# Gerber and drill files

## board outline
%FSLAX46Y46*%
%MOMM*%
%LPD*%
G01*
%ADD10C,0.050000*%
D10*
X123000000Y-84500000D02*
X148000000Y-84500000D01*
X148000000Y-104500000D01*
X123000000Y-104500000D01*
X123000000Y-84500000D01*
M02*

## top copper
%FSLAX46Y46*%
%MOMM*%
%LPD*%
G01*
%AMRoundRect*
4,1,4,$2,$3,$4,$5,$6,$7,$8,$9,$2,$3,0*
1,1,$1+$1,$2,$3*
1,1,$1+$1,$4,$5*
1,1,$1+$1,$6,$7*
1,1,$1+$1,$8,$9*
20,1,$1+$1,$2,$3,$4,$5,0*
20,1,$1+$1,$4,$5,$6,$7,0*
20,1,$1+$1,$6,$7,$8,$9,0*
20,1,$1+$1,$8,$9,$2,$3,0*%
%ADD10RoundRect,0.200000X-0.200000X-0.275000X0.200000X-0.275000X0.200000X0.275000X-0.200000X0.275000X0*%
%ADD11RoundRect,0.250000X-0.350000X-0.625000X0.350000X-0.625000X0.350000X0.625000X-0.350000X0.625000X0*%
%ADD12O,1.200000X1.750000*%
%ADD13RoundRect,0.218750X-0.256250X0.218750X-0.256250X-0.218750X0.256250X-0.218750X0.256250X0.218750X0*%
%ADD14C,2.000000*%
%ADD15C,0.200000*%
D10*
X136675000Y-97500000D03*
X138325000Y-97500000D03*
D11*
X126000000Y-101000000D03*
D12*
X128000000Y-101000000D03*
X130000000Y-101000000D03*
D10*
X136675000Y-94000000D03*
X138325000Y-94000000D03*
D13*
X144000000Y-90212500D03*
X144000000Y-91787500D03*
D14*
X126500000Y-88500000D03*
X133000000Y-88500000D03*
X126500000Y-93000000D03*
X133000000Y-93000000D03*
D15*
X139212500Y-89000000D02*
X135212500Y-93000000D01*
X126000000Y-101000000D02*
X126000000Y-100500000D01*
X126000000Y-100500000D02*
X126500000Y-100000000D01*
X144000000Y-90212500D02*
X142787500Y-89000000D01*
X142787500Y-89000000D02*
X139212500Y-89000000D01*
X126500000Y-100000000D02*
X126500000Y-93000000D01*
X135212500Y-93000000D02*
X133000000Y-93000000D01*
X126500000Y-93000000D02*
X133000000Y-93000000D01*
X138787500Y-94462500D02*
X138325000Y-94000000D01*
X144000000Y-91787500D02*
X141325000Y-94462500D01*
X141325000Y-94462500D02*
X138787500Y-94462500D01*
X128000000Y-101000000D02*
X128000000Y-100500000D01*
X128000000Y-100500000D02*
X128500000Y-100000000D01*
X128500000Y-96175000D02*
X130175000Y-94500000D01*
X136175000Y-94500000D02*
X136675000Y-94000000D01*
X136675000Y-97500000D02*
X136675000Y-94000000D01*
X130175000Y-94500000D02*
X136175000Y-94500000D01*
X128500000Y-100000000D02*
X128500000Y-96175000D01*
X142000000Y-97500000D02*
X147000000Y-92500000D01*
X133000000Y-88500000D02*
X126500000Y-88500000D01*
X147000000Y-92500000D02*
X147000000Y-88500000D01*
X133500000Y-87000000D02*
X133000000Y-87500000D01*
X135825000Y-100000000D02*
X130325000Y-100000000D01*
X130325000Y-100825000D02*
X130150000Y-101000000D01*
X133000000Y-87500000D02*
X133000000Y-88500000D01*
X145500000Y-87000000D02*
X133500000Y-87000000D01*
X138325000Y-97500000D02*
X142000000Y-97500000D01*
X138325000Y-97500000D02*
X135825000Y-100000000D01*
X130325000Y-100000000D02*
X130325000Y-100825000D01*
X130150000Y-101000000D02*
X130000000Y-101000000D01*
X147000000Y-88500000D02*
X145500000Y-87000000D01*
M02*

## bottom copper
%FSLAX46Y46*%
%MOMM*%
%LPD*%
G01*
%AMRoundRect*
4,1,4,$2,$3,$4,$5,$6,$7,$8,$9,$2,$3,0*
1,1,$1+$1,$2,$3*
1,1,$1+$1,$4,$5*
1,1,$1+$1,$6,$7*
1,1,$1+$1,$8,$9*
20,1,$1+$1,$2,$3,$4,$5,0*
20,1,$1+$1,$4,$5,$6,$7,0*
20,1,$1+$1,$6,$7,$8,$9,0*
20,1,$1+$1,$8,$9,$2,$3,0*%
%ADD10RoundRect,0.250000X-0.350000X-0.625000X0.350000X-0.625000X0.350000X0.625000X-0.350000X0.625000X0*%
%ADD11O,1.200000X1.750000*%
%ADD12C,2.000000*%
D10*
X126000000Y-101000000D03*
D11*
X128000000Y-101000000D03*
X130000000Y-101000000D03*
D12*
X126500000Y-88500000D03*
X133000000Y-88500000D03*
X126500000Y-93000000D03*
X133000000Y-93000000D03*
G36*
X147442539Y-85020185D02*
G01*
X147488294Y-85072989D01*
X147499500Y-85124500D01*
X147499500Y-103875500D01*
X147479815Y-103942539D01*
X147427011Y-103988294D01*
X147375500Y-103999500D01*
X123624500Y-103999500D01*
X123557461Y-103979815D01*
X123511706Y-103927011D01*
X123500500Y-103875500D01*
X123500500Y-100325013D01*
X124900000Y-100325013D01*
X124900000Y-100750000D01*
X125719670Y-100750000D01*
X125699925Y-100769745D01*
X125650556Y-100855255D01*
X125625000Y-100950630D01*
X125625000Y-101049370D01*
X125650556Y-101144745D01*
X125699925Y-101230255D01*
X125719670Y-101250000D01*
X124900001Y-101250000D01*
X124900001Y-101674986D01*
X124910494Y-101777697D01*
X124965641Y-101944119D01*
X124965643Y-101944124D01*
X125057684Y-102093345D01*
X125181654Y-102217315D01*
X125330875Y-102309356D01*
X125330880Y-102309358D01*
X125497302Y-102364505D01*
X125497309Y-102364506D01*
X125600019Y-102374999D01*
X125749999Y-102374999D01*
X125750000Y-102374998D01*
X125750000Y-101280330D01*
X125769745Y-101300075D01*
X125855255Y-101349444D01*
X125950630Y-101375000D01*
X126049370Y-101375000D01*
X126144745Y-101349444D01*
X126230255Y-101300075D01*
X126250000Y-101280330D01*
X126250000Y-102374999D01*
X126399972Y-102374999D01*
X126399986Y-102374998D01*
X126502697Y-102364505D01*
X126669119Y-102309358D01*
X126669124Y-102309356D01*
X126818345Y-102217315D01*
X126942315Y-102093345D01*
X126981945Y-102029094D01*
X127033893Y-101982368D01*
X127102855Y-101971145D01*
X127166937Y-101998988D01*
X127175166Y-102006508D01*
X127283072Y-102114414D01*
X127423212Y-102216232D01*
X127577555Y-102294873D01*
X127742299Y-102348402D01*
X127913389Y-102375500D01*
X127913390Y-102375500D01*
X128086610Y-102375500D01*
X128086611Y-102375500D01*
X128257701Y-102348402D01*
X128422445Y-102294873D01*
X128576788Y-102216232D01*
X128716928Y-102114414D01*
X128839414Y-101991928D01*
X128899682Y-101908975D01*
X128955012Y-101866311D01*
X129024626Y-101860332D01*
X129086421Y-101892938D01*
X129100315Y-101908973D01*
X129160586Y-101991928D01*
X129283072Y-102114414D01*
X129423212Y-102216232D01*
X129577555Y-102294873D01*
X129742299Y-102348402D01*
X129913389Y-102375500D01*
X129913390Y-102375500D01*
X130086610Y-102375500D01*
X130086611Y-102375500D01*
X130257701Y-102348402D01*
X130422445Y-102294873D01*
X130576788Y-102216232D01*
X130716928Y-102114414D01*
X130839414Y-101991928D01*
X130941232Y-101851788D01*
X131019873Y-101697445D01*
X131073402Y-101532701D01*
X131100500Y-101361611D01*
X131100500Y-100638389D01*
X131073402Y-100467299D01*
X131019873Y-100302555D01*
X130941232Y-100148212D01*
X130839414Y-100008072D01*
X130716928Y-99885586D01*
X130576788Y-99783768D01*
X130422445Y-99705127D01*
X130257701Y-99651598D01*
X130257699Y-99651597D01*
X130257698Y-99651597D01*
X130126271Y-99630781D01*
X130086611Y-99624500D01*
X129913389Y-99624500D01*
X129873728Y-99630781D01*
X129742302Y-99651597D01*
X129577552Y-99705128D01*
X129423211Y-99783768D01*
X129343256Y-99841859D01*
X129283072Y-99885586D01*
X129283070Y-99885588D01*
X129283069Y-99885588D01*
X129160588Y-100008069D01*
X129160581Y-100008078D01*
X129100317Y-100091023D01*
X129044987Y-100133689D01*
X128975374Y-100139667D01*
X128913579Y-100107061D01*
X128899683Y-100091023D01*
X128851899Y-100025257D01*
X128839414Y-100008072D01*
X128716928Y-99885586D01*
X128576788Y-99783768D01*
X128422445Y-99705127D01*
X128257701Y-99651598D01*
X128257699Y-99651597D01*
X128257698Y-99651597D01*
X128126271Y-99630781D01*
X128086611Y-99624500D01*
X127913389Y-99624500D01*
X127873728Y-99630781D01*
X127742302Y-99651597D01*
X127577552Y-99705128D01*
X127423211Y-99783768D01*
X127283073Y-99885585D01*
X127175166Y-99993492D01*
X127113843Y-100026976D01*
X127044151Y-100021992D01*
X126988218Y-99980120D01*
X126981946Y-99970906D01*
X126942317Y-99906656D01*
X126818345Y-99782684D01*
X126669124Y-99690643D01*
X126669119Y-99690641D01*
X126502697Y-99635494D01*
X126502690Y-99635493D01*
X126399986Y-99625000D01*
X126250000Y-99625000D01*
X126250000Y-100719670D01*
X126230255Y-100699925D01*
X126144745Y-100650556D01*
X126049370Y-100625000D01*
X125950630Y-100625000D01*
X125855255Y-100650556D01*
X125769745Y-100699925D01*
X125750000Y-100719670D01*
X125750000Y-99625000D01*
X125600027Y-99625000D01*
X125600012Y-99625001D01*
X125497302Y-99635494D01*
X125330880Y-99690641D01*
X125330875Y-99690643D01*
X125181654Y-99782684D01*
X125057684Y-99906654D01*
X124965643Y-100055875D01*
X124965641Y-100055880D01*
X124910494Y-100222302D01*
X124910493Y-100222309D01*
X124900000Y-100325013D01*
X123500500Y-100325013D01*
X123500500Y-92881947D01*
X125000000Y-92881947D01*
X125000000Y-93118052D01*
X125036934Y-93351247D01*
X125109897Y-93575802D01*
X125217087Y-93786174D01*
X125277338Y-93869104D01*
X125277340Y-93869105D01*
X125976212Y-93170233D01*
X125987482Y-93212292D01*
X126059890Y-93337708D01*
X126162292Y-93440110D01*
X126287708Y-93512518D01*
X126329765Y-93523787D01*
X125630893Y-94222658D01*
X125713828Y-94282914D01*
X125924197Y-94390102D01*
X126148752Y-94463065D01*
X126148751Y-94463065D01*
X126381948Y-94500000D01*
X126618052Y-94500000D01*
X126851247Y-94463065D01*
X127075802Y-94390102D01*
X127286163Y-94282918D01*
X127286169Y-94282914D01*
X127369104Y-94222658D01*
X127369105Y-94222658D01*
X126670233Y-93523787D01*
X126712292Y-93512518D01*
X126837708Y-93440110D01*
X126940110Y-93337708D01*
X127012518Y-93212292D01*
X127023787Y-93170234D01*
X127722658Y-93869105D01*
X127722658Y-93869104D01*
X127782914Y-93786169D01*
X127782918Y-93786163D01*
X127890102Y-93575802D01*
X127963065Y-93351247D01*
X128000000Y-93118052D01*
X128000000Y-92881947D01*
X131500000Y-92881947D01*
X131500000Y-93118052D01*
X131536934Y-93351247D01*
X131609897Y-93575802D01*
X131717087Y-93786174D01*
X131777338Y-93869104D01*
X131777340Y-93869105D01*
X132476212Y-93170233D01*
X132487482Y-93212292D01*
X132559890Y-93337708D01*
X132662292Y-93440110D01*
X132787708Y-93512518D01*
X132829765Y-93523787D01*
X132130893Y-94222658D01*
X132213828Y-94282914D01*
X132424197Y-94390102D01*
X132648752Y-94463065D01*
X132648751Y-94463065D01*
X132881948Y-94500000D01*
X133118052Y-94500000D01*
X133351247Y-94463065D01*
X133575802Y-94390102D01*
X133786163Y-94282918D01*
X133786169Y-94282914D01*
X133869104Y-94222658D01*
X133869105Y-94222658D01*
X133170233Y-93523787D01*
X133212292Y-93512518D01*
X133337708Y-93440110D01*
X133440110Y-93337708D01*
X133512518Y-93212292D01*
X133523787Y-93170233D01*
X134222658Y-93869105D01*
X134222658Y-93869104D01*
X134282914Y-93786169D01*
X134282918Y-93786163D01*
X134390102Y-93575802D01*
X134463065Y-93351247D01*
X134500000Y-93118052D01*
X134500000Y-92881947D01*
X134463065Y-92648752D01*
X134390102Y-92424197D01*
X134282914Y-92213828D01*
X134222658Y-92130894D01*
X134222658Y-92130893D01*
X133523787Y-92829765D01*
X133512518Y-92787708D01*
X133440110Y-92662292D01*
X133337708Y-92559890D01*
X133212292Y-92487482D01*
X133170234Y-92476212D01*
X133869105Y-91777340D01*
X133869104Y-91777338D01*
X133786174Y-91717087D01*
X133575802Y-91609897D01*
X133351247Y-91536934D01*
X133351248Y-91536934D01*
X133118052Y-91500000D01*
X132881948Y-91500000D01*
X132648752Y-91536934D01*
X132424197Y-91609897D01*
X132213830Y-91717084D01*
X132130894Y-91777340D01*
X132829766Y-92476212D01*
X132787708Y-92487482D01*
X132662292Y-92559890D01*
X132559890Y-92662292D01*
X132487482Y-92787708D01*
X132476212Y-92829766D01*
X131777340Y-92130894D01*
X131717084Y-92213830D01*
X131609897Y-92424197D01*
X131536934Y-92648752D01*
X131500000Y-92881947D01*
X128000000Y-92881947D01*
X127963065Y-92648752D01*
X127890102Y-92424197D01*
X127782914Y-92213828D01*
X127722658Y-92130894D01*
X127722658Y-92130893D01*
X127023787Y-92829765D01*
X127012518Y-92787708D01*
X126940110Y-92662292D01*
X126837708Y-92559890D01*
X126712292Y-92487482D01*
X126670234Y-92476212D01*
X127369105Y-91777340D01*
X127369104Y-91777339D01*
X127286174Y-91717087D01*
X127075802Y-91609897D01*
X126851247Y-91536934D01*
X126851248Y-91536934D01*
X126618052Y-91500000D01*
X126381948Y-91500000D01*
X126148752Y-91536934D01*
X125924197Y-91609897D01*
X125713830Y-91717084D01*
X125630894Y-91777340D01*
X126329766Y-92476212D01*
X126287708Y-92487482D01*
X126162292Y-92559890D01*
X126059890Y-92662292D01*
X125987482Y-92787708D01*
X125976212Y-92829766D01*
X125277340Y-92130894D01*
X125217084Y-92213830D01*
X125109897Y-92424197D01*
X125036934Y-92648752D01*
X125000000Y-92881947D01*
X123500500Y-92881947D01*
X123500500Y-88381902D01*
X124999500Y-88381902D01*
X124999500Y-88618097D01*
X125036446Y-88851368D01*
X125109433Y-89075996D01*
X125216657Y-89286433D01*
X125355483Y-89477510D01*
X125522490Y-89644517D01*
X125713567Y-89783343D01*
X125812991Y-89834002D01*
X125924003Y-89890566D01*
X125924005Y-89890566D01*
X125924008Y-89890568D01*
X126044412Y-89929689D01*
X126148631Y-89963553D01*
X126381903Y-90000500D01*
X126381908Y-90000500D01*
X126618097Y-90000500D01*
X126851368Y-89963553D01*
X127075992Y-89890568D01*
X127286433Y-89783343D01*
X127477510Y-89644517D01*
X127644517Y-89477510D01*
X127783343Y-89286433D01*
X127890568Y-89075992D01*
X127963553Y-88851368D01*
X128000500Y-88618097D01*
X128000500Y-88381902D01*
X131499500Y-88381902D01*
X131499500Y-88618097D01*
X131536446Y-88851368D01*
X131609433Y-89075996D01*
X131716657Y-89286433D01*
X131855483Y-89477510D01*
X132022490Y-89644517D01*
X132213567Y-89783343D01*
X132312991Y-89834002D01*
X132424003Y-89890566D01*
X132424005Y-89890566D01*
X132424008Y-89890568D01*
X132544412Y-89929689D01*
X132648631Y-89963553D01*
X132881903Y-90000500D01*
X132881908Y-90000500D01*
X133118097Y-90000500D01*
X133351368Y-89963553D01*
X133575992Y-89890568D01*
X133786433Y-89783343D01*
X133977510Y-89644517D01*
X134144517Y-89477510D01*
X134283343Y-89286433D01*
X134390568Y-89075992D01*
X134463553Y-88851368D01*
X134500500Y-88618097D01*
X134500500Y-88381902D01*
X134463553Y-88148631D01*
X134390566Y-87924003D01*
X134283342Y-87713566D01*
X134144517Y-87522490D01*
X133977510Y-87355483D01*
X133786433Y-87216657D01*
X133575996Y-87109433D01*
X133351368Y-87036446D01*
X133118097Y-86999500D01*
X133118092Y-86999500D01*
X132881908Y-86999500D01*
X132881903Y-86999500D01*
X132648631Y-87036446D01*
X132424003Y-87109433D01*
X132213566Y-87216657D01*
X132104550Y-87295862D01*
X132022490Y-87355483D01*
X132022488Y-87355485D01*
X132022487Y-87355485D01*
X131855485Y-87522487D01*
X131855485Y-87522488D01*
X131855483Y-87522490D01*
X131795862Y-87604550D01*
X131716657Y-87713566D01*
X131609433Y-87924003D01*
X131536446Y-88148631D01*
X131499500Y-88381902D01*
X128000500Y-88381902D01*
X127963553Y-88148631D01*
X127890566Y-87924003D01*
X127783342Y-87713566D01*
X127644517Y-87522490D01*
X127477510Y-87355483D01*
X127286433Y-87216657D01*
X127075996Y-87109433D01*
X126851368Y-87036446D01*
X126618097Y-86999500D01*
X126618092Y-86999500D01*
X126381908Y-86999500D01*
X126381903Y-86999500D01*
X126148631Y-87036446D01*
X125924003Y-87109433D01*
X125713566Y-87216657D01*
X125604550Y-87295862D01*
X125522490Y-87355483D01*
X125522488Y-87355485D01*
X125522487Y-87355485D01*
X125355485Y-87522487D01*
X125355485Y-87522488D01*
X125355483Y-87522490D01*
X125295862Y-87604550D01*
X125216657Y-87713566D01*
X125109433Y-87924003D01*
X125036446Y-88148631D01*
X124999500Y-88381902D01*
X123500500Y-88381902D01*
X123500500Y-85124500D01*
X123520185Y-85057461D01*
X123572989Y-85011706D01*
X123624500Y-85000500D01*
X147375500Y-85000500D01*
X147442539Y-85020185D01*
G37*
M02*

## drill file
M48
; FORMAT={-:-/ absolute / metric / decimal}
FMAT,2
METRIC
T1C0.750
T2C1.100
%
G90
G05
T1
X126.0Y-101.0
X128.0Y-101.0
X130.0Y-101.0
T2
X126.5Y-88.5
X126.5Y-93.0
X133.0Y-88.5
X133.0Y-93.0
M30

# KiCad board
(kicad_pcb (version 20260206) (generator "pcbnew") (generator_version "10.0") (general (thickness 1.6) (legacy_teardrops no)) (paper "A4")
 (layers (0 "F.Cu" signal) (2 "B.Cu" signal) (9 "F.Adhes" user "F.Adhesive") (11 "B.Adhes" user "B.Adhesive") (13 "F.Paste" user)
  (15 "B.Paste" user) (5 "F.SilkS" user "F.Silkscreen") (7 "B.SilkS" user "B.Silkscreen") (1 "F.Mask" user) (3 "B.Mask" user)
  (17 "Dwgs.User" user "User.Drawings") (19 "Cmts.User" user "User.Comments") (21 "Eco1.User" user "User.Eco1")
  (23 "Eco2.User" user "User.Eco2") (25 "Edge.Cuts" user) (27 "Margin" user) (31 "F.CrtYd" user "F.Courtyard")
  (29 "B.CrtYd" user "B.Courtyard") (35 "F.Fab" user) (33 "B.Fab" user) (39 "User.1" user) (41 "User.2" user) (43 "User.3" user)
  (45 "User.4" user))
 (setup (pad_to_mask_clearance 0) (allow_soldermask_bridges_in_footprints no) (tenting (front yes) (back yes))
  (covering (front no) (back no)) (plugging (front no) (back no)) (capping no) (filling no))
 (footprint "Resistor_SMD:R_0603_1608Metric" (layer "F.Cu") (at 137.5 97.5)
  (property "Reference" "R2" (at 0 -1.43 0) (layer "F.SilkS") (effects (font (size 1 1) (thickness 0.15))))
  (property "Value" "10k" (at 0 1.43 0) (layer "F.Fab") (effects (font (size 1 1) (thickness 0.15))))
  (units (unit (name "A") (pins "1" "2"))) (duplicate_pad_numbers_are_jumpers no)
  (pad "1" smd roundrect (at -0.825 0) (size 0.8 0.95) (layers "F.Cu" "F.Mask" "F.Paste") (roundrect_rratio 0.25) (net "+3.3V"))
  (pad "2" smd roundrect (at 0.825 0) (size 0.8 0.95) (layers "F.Cu" "F.Mask" "F.Paste") (roundrect_rratio 0.25) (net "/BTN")))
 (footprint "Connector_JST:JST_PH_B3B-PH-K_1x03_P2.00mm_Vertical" (layer "F.Cu") (at 126 101)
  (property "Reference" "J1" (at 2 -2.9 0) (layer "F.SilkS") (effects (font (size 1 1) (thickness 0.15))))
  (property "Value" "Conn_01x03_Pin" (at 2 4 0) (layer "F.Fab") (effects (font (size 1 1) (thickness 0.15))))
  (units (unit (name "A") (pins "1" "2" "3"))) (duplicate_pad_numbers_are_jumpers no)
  (pad "1" thru_hole roundrect (at 0 0) (size 1.2 1.75) (drill 0.75) (layers "*.Cu" "*.Mask") (remove_unused_layers no)
   (roundrect_rratio 0.208333) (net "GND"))
  (pad "2" thru_hole oval (at 2 0) (size 1.2 1.75) (drill 0.75) (layers "*.Cu" "*.Mask") (remove_unused_layers no) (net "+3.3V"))
  (pad "3" thru_hole oval (at 4 0) (size 1.2 1.75) (drill 0.75) (layers "*.Cu" "*.Mask") (remove_unused_layers no) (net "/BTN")))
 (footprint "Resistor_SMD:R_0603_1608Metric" (layer "F.Cu") (at 137.5 94)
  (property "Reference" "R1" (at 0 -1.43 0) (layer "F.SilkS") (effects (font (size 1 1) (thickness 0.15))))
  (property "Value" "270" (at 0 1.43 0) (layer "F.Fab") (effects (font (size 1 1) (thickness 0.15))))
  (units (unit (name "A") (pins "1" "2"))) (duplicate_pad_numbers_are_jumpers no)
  (pad "1" smd roundrect (at -0.825 0) (size 0.8 0.95) (layers "F.Cu" "F.Mask" "F.Paste") (roundrect_rratio 0.25) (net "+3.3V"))
  (pad "2" smd roundrect (at 0.825 0) (size 0.8 0.95) (layers "F.Cu" "F.Mask" "F.Paste") (roundrect_rratio 0.25) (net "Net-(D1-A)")))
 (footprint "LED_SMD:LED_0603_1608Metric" (layer "F.Cu") (at 144 91 -90)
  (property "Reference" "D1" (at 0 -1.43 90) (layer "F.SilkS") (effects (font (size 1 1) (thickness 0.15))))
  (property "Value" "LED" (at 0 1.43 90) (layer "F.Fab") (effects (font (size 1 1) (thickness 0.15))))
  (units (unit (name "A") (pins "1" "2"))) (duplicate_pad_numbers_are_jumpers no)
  (pad "1" smd roundrect (at -0.7875 0 270) (size 0.875 0.95) (layers "F.Cu" "F.Mask" "F.Paste") (roundrect_rratio 0.25) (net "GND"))
  (pad "2" smd roundrect (at 0.7875 0 270) (size 0.875 0.95) (layers "F.Cu" "F.Mask" "F.Paste") (roundrect_rratio 0.25) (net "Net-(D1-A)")))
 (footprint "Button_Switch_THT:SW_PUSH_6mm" (layer "F.Cu") (at 126.5 88.5)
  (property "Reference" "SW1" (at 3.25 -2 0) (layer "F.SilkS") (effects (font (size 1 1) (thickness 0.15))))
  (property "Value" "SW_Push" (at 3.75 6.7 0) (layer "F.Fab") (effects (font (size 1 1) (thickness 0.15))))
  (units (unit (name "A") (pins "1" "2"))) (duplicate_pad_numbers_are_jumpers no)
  (pad "1" thru_hole circle (at 0 0 90) (size 2 2) (drill 1.1) (layers "*.Cu" "*.Mask") (remove_unused_layers no) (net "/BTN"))
  (pad "1" thru_hole circle (at 6.5 0 90) (size 2 2) (drill 1.1) (layers "*.Cu" "*.Mask") (remove_unused_layers no) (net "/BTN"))
  (pad "2" thru_hole circle (at 0 4.5 90) (size 2 2) (drill 1.1) (layers "*.Cu" "*.Mask") (remove_unused_layers no) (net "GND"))
  (pad "2" thru_hole circle (at 6.5 4.5 90) (size 2 2) (drill 1.1) (layers "*.Cu" "*.Mask") (remove_unused_layers no) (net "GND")))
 (gr_rect (start 123 84.5) (end 148 104.5) (stroke (width 0.05) (type default)) (fill no) (layer "Edge.Cuts"))
 (segment (start 139.2125 89) (end 135.2125 93) (width 0.2) (layer "F.Cu") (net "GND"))
 (segment (start 126 101) (end 126 100.5) (width 0.2) (layer "F.Cu") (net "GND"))
 (segment (start 126 100.5) (end 126.5 100) (width 0.2) (layer "F.Cu") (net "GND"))
 (segment (start 144 90.2125) (end 142.7875 89) (width 0.2) (layer "F.Cu") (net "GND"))
 (segment (start 142.7875 89) (end 139.2125 89) (width 0.2) (layer "F.Cu") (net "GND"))
 (segment (start 126.5 100) (end 126.5 93) (width 0.2) (layer "F.Cu") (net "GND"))
 (segment (start 135.2125 93) (end 133 93) (width 0.2) (layer "F.Cu") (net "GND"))
 (segment (start 126.5 93) (end 133 93) (width 0.2) (layer "F.Cu") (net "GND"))
 (segment (start 138.7875 94.4625) (end 138.325 94) (width 0.2) (layer "F.Cu") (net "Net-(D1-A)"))
 (segment (start 144 91.7875) (end 141.325 94.4625) (width 0.2) (layer "F.Cu") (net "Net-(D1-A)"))
 (segment (start 141.325 94.4625) (end 138.7875 94.4625) (width 0.2) (layer "F.Cu") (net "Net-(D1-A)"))
 (segment (start 128 101) (end 128 100.5) (width 0.2) (layer "F.Cu") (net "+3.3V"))
 (segment (start 128 100.5) (end 128.5 100) (width 0.2) (layer "F.Cu") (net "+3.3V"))
 (segment (start 128.5 96.175) (end 130.175 94.5) (width 0.2) (layer "F.Cu") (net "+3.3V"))
 (segment (start 136.175 94.5) (end 136.675 94) (width 0.2) (layer "F.Cu") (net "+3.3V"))
 (segment (start 136.675 97.5) (end 136.675 94) (width 0.2) (layer "F.Cu") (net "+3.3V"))
 (segment (start 130.175 94.5) (end 136.175 94.5) (width 0.2) (layer "F.Cu") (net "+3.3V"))
 (segment (start 128.5 100) (end 128.5 96.175) (width 0.2) (layer "F.Cu") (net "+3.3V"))
 (segment (start 142 97.5) (end 147 92.5) (width 0.2) (layer "F.Cu") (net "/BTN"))
 (segment (start 133 88.5) (end 126.5 88.5) (width 0.2) (layer "F.Cu") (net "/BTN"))
 (segment (start 147 92.5) (end 147 88.5) (width 0.2) (layer "F.Cu") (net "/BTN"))
 (segment (start 133.5 87) (end 133 87.5) (width 0.2) (layer "F.Cu") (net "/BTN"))
 (segment (start 135.825 100) (end 130.325 100) (width 0.2) (layer "F.Cu") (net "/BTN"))
 (segment (start 130.325 100.825) (end 130.15 101) (width 0.2) (layer "F.Cu") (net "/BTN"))
 (segment (start 133 87.5) (end 133 88.5) (width 0.2) (layer "F.Cu") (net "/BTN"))
 (segment (start 145.5 87) (end 133.5 87) (width 0.2) (layer "F.Cu") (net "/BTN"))
 (segment (start 138.325 97.5) (end 142 97.5) (width 0.2) (layer "F.Cu") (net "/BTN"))
 (segment (start 138.325 97.5) (end 135.825 100) (width 0.2) (layer "F.Cu") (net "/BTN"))
 (segment (start 130.325 100) (end 130.325 100.825) (width 0.2) (layer "F.Cu") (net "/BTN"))
 (segment (start 130.15 101) (end 130 101) (width 0.2) (layer "F.Cu") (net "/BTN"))
 (segment (start 147 88.5) (end 145.5 87) (width 0.2) (layer "F.Cu") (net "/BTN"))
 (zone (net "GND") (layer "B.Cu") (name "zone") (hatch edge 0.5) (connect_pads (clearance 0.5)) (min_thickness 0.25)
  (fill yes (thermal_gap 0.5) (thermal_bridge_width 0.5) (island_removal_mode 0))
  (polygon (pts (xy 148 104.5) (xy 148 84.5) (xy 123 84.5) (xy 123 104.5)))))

